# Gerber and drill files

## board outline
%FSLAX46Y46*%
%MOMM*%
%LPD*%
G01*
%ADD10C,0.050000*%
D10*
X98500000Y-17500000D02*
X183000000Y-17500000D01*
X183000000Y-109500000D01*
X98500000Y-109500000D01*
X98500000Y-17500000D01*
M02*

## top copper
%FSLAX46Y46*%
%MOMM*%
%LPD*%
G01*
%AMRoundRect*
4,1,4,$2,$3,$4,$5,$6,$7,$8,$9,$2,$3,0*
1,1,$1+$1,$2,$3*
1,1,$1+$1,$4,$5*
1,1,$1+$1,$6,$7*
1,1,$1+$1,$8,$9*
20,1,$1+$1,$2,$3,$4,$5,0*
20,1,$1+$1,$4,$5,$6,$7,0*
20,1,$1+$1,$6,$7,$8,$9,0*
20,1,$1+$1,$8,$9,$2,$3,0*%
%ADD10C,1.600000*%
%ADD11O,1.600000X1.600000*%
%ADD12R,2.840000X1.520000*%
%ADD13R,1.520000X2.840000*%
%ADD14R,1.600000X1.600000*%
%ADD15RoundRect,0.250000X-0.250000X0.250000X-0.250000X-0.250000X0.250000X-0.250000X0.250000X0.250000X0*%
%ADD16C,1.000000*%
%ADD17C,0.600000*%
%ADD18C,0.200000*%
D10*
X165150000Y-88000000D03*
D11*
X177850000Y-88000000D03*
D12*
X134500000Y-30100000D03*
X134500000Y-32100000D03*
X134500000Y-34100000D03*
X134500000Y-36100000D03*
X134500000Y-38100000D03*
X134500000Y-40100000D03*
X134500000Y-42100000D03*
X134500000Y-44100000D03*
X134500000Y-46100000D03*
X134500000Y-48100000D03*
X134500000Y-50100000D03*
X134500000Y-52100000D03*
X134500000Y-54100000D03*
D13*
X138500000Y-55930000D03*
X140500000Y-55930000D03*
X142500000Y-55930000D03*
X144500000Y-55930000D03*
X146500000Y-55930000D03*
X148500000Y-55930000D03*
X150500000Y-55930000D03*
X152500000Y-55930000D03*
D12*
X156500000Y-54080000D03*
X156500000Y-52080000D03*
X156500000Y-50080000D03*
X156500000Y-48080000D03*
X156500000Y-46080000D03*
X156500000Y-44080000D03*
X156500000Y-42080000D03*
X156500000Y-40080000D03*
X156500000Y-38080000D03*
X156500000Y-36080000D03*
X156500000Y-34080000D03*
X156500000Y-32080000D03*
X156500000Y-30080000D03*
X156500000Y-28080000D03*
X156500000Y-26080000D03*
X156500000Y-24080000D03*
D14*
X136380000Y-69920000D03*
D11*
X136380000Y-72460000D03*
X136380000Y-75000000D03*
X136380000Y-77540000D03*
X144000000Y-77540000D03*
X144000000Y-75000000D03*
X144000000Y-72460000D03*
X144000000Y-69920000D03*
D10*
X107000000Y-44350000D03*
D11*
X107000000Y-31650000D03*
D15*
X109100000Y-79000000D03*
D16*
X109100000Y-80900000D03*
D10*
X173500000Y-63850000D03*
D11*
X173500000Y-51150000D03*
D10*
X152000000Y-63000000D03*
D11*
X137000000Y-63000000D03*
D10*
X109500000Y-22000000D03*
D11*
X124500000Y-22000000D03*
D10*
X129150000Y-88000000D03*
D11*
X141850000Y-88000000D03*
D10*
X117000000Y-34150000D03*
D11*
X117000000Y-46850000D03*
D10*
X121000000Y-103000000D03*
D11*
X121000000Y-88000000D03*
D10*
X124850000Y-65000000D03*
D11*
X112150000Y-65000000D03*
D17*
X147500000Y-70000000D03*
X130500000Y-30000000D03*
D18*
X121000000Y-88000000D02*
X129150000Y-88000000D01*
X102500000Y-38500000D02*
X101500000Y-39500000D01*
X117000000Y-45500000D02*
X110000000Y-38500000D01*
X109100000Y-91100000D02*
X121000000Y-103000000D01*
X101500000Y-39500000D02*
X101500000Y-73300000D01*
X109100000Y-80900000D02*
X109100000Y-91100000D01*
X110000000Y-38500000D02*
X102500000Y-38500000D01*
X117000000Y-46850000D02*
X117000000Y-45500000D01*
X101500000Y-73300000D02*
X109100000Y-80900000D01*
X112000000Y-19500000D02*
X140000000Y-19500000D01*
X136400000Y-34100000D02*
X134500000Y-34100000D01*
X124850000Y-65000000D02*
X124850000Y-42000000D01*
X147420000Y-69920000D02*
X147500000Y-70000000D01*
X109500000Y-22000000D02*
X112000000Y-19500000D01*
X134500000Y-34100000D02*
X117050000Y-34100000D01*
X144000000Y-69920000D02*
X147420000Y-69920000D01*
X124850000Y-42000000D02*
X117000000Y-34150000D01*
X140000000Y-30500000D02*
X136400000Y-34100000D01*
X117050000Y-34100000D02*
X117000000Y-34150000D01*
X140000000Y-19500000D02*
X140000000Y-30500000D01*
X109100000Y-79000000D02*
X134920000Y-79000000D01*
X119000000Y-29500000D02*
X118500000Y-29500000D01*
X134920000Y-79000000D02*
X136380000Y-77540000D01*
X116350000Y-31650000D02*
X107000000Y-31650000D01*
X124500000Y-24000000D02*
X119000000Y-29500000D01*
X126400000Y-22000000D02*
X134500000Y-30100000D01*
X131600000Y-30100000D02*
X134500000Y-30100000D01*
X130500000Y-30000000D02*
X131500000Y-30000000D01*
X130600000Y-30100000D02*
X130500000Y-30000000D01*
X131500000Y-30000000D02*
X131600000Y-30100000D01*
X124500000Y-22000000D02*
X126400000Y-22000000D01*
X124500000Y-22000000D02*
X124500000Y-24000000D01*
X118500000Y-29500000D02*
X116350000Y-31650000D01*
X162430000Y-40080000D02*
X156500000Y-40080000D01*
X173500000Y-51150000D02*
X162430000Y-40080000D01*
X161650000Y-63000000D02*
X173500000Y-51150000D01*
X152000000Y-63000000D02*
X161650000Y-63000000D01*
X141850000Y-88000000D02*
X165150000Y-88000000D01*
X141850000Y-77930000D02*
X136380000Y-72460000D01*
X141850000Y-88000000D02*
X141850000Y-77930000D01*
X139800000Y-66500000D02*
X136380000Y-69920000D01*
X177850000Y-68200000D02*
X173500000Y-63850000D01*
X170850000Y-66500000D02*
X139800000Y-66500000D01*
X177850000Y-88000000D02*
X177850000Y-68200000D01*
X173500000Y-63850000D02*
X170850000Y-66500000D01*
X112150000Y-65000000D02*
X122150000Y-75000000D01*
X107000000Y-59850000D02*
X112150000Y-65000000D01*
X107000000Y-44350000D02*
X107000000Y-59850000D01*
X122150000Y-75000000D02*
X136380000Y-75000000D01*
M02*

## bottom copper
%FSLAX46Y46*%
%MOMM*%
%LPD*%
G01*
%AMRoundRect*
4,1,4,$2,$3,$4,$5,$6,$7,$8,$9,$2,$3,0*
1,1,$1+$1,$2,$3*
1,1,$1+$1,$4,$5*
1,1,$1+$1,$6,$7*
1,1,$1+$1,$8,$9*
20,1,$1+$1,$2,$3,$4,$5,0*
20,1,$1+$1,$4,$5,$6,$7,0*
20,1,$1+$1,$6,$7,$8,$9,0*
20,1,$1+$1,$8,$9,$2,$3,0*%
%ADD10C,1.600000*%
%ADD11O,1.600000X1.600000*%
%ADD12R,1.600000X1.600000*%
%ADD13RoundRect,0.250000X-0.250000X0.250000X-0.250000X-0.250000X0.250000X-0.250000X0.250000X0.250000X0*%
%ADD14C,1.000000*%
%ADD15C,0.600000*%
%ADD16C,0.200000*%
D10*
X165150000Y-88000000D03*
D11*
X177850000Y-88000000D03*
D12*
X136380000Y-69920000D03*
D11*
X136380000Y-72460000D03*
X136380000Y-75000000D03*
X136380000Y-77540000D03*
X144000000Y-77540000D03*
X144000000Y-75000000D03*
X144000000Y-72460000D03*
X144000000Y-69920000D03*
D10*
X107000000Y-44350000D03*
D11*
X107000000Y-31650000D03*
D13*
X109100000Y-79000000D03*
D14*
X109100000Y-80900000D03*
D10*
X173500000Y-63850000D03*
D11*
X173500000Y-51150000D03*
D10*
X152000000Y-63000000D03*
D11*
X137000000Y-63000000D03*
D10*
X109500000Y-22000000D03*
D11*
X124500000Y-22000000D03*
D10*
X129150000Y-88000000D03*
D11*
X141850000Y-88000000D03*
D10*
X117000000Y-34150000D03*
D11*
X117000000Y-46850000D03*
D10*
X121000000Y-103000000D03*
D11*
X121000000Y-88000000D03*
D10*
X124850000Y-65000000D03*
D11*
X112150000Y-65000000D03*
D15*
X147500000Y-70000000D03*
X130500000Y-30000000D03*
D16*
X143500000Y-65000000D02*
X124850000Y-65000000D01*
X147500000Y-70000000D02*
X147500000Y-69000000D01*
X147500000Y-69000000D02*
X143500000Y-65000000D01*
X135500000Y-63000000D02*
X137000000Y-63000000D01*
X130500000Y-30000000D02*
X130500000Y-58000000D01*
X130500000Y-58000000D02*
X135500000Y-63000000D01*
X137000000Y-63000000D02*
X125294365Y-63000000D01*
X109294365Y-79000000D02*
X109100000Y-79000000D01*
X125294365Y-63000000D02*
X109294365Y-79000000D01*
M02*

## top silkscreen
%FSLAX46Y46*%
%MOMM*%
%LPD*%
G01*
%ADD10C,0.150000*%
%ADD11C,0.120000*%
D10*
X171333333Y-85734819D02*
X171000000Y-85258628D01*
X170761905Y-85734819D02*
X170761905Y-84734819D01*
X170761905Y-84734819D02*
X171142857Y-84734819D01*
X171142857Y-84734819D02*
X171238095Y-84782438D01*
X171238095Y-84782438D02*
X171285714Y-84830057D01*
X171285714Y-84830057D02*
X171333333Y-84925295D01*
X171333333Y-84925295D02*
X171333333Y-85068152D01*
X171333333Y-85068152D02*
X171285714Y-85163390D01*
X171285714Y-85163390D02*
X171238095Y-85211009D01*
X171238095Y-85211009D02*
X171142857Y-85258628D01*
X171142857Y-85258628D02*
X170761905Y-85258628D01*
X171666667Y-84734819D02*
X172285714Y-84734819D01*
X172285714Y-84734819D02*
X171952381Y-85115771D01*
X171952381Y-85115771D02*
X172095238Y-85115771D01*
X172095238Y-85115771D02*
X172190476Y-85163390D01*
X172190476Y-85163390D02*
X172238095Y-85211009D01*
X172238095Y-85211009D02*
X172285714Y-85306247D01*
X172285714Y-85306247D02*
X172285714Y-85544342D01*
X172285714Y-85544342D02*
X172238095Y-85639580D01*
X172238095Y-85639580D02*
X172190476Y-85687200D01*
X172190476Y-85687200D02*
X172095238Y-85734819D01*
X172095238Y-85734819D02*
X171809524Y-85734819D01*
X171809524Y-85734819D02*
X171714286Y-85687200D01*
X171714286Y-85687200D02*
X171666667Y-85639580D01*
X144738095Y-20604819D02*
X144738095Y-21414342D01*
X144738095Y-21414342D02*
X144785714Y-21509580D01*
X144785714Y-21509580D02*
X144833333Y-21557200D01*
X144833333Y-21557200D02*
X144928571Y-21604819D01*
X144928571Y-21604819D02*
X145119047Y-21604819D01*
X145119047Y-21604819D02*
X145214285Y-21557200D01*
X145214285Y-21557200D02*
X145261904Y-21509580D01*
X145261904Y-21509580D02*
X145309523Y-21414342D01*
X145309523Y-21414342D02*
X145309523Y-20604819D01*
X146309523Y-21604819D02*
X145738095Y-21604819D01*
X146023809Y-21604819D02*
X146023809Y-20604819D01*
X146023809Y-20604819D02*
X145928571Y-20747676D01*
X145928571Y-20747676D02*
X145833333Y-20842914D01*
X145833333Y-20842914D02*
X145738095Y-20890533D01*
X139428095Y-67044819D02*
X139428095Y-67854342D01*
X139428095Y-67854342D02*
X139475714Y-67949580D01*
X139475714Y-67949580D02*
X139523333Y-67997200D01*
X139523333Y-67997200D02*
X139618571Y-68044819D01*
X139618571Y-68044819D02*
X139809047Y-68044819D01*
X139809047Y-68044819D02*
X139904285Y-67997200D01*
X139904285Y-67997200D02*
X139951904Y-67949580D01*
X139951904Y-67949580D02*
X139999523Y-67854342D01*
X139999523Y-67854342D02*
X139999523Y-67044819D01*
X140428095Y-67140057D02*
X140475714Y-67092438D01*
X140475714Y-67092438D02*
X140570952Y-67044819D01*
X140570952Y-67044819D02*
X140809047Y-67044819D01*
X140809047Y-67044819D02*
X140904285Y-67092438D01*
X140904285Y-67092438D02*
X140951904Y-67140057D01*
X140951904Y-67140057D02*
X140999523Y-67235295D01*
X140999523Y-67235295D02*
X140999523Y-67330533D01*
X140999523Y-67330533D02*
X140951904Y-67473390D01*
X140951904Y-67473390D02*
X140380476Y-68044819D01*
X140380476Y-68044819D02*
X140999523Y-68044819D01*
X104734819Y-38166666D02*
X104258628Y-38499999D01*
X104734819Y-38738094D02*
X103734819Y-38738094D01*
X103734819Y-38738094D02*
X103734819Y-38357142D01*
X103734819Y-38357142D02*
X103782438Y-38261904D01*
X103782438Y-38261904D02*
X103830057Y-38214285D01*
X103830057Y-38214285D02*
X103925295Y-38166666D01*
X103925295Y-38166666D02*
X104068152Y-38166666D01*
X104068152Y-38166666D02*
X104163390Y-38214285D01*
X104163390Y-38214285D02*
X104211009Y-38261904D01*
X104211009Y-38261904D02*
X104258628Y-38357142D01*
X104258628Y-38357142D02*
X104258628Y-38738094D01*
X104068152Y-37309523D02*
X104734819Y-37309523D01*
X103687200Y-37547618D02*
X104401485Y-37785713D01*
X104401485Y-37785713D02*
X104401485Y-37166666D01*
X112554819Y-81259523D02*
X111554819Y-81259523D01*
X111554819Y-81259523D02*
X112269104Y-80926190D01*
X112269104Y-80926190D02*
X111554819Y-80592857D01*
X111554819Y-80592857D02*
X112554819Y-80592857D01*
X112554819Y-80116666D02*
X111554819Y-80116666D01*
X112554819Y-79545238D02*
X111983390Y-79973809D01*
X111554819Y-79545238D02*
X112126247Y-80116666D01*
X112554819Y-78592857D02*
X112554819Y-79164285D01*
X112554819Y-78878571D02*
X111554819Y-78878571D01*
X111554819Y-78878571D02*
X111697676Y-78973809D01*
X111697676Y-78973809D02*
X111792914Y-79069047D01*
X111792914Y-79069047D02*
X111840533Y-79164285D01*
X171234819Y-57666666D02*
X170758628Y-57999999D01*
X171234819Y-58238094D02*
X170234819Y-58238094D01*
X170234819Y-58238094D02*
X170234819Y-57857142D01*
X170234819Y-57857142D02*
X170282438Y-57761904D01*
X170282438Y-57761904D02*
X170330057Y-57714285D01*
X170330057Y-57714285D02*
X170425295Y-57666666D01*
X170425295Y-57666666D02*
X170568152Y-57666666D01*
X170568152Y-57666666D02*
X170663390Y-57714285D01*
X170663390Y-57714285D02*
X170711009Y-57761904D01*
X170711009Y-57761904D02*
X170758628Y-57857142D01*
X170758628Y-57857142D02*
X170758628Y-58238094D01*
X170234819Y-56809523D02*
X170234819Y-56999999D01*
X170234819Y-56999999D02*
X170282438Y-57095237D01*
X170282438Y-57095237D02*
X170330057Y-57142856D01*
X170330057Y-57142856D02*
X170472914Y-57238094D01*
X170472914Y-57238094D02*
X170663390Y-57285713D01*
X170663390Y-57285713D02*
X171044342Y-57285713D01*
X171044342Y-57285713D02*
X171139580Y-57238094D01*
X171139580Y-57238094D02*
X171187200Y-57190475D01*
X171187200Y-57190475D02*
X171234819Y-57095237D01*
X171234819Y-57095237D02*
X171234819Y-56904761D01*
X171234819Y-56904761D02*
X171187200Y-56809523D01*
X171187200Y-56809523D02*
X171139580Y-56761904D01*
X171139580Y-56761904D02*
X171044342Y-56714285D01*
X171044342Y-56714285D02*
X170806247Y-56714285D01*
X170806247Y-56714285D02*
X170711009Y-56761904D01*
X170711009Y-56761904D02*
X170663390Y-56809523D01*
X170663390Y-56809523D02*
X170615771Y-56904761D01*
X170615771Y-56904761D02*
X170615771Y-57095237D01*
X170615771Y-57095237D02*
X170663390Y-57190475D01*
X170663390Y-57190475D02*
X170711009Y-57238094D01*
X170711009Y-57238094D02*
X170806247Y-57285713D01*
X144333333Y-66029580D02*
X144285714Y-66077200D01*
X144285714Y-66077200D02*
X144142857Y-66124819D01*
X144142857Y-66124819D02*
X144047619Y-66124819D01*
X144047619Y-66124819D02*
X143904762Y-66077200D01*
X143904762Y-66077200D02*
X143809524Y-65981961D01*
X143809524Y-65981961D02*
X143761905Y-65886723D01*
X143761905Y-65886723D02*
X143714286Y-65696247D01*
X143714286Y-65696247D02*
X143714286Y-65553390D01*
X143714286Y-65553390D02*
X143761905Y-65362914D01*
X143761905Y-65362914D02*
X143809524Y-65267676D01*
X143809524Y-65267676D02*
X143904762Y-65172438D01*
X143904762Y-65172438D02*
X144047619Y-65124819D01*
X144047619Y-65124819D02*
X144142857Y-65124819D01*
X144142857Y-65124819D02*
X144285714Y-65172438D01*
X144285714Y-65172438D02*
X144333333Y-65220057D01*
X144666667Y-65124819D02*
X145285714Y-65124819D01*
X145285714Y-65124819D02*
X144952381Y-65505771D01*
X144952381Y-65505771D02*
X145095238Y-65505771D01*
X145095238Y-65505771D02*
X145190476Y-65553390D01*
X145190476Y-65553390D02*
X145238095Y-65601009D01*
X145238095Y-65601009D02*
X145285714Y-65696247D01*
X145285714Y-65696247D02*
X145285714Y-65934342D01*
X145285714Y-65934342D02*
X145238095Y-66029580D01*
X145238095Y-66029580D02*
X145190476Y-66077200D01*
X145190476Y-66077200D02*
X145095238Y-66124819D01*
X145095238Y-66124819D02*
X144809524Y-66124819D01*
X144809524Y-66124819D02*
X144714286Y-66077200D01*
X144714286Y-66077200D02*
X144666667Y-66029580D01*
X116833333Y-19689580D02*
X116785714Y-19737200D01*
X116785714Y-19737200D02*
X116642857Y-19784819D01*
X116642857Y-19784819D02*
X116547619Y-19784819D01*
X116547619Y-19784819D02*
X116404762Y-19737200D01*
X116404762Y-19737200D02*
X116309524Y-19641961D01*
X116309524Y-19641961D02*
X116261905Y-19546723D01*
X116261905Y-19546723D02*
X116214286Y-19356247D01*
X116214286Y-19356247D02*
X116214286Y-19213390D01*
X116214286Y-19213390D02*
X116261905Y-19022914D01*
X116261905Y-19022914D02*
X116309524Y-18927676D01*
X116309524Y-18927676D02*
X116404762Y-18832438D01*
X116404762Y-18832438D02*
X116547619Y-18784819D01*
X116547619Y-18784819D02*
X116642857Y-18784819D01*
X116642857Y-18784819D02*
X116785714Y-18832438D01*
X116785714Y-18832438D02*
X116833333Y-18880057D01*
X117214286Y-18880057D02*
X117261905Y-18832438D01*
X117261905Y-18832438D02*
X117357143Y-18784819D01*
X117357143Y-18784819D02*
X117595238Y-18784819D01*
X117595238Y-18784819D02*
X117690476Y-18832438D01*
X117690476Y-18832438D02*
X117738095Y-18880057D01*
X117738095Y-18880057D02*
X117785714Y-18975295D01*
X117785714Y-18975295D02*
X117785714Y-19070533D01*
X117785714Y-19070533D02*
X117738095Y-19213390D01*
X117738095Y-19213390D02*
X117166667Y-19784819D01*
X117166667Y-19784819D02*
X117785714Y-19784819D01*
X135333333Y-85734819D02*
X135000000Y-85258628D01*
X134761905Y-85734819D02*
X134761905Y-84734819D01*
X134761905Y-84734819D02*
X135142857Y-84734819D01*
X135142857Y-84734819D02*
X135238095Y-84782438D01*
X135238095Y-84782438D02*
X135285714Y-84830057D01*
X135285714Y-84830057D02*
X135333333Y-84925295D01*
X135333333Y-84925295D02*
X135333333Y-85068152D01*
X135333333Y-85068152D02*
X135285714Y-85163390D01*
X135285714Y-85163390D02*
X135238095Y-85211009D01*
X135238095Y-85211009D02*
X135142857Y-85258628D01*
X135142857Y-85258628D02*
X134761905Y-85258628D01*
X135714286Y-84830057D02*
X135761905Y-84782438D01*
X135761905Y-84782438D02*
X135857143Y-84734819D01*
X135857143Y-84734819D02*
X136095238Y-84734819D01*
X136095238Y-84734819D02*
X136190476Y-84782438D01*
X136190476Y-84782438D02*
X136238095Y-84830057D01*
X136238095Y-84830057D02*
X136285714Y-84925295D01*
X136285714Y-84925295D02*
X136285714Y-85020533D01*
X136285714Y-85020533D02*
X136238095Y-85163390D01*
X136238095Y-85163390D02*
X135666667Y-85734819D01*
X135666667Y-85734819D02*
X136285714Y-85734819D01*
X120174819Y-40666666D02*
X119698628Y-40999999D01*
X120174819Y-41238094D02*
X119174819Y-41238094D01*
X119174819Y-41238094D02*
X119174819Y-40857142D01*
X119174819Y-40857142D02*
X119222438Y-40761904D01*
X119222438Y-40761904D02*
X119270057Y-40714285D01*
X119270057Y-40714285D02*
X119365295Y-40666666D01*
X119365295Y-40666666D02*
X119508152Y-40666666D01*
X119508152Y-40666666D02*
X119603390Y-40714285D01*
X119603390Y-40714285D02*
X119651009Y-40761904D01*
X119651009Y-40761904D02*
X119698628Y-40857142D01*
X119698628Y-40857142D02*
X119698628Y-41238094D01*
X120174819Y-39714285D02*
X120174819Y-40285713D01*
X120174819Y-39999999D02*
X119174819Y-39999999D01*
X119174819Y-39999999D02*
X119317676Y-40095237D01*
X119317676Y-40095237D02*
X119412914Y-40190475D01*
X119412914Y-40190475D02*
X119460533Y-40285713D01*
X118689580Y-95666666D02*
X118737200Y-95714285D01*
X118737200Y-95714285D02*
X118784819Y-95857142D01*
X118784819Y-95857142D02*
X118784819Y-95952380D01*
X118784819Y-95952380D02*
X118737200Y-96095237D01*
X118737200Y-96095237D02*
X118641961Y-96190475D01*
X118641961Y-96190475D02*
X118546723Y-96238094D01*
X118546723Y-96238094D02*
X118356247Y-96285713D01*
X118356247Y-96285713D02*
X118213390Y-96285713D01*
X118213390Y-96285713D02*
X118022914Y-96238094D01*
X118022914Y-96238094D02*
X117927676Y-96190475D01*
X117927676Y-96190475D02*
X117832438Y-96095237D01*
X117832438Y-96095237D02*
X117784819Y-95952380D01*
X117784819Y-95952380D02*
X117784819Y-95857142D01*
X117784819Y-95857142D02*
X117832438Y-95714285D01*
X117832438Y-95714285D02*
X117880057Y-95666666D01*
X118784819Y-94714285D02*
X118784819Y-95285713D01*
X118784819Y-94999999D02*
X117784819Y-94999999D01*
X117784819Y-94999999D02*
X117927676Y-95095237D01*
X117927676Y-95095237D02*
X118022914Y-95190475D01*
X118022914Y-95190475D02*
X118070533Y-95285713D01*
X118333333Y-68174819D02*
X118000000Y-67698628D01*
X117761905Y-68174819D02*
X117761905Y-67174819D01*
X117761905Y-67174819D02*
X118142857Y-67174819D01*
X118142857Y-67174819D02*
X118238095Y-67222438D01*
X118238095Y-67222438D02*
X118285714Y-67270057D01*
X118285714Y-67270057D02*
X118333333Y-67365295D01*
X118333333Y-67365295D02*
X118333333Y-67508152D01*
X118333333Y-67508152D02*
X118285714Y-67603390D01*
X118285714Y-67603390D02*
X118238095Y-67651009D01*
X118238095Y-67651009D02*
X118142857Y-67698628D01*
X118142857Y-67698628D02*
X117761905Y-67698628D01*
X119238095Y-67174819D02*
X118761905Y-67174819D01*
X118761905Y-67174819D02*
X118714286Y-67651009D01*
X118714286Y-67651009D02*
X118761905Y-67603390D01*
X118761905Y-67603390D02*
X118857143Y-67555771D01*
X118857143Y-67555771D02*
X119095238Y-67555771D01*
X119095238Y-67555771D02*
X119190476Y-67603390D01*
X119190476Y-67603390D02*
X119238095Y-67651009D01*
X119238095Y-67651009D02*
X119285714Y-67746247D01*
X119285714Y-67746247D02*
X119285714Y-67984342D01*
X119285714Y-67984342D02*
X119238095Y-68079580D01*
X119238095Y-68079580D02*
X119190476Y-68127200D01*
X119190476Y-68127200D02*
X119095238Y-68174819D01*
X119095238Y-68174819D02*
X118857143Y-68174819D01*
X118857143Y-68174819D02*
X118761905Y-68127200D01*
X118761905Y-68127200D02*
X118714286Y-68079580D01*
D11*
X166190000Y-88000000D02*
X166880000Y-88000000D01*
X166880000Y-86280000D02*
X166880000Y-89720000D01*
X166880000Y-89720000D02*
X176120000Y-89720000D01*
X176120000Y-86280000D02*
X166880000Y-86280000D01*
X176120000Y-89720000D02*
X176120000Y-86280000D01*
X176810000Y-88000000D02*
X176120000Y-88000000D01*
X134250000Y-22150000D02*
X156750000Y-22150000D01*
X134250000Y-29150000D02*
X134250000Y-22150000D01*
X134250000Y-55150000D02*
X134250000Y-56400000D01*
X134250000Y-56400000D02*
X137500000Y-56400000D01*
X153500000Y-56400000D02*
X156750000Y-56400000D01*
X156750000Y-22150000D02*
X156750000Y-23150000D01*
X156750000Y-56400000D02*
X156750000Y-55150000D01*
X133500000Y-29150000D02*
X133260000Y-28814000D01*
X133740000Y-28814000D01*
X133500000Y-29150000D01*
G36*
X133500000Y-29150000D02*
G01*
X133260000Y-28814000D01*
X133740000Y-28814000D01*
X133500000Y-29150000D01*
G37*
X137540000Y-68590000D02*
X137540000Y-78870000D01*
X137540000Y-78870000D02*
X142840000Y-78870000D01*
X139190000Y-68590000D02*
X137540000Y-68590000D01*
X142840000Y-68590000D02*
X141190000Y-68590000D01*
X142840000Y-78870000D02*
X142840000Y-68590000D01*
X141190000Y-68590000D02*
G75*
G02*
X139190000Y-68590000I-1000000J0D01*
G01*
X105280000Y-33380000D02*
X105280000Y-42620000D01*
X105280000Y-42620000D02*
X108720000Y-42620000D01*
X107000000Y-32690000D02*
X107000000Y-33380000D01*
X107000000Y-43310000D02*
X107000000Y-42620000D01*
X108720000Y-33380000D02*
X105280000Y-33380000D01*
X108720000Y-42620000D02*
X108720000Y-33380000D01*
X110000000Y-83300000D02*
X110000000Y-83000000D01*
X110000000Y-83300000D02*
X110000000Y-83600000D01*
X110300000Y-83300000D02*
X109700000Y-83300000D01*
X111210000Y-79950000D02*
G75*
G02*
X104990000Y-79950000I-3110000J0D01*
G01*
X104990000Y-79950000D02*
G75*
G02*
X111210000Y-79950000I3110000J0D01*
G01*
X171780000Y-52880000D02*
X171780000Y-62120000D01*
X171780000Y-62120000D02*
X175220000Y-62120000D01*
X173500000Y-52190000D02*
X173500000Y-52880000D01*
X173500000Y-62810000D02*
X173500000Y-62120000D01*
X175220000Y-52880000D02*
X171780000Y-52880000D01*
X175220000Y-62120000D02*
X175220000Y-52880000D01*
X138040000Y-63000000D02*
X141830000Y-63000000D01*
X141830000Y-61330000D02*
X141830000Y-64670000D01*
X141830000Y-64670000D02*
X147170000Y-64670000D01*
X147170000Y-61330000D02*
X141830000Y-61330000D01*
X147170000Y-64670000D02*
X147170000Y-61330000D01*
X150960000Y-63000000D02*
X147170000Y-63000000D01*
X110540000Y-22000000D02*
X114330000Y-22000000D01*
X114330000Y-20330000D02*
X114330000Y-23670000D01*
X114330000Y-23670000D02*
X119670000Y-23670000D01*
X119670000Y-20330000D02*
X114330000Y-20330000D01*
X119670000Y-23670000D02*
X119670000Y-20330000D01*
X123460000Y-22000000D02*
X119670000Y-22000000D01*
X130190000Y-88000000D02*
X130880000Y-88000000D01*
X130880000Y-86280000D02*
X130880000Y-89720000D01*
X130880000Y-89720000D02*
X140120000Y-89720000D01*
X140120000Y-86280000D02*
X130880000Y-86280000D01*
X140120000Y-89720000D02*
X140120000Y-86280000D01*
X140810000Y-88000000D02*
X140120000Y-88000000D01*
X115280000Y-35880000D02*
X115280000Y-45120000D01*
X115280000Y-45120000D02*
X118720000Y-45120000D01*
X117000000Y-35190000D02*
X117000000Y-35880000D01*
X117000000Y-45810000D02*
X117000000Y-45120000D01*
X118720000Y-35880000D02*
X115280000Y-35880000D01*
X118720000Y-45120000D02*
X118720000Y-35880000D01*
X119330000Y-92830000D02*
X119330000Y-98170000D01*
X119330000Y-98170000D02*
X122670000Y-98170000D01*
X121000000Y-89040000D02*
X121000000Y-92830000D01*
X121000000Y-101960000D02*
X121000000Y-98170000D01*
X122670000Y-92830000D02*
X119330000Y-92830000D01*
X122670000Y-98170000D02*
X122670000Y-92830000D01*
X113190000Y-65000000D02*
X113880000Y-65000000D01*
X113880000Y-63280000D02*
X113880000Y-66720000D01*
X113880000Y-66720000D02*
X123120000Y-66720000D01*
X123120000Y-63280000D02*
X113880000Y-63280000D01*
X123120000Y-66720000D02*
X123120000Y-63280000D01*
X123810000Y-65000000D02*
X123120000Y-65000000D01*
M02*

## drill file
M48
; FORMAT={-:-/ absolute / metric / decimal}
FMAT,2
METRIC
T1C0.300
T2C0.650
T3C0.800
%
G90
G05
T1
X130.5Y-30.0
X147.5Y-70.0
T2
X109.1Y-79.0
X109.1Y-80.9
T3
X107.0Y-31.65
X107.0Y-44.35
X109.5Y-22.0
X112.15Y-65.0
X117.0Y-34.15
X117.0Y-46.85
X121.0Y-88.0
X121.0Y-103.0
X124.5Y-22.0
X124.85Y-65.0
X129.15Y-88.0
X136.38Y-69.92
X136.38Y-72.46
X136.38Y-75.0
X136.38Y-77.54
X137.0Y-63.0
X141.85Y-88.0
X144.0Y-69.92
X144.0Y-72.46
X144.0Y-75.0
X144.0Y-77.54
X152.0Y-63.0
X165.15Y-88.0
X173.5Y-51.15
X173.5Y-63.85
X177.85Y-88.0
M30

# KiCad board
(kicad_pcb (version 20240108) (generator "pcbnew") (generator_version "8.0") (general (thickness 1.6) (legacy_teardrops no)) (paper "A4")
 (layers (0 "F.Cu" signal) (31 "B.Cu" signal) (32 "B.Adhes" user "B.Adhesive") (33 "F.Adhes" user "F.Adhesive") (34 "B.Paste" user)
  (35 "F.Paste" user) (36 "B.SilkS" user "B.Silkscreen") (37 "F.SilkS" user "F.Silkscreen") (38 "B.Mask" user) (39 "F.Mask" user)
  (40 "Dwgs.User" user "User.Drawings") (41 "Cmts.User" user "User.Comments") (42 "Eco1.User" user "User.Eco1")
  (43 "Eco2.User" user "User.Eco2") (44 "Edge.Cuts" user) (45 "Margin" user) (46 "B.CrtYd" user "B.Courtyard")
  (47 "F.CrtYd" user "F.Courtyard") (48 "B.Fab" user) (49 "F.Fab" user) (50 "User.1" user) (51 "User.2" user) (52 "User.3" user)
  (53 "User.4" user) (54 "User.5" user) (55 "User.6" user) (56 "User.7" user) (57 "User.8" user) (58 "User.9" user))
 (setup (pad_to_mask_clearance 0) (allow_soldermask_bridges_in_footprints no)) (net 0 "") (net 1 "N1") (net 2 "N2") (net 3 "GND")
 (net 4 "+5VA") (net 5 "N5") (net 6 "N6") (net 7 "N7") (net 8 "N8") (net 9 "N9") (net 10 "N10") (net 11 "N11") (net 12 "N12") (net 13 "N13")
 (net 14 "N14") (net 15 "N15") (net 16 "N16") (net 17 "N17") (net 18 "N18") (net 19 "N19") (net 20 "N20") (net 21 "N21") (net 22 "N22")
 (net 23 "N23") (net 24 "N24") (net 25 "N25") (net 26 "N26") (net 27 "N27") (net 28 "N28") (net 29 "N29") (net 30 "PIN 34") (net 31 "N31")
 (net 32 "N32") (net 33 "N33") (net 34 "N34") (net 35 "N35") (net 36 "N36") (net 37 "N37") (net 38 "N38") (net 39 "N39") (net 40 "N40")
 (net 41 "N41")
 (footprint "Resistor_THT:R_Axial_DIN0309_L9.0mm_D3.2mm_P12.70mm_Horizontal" (layer "F.Cu") (at 165.15 88)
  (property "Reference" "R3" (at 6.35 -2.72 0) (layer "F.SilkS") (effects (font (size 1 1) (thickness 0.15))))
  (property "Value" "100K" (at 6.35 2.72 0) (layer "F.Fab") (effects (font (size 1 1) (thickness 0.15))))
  (fp_line (start 1.04 0) (end 1.73 0) (stroke (width 0.12) (type solid)) (layer "F.SilkS"))
  (fp_line (start 1.73 -1.72) (end 1.73 1.72) (stroke (width 0.12) (type solid)) (layer "F.SilkS"))
  (fp_line (start 1.73 1.72) (end 10.97 1.72) (stroke (width 0.12) (type solid)) (layer "F.SilkS"))
  (fp_line (start 10.97 -1.72) (end 1.73 -1.72) (stroke (width 0.12) (type solid)) (layer "F.SilkS"))
  (fp_line (start 10.97 1.72) (end 10.97 -1.72) (stroke (width 0.12) (type solid)) (layer "F.SilkS"))
  (fp_line (start 11.66 0) (end 10.97 0) (stroke (width 0.12) (type solid)) (layer "F.SilkS"))
  (pad "1" thru_hole circle (at 0 0) (size 1.6 1.6) (drill 0.8) (layers "*.Cu" "*.Mask") (remove_unused_layers no) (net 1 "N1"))
  (pad "2" thru_hole oval (at 12.7 0) (size 1.6 1.6) (drill 0.8) (layers "*.Cu" "*.Mask") (remove_unused_layers no) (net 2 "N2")))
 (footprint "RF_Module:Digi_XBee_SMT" (layer "F.Cu") (at 145.5 40)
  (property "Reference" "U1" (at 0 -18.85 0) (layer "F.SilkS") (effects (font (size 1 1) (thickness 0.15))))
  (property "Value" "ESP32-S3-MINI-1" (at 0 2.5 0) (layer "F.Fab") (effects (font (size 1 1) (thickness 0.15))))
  (fp_line (start -11.25 -17.85) (end 11.25 -17.85) (stroke (width 0.12) (type solid)) (layer "F.SilkS"))
  (fp_line (start -11.25 -10.85) (end -11.25 -17.85) (stroke (width 0.12) (type solid)) (layer "F.SilkS"))
  (fp_line (start -11.25 15.15) (end -11.25 16.4) (stroke (width 0.12) (type solid)) (layer "F.SilkS"))
  (fp_line (start -11.25 16.4) (end -8 16.4) (stroke (width 0.12) (type solid)) (layer "F.SilkS"))
  (fp_line (start 8 16.4) (end 11.25 16.4) (stroke (width 0.12) (type solid)) (layer "F.SilkS"))
  (fp_line (start 11.25 -17.85) (end 11.25 -16.85) (stroke (width 0.12) (type solid)) (layer "F.SilkS"))
  (fp_line (start 11.25 16.4) (end 11.25 15.15) (stroke (width 0.12) (type solid)) (layer "F.SilkS"))
  (fp_poly
   (pts (xy -12 -10.85) (xy -12.24 -11.186) (xy -11.76 -11.186) (xy -12 -10.85)) (stroke (width 0.12) (type solid)) (fill solid)
   (layer "F.SilkS"))
  (pad "1" smd rect (at -11 -9.9) (size 2.84 1.52) (layers "F.Cu" "F.Paste" "F.Mask") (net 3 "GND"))
  (pad "2" smd rect (at -11 -7.9) (size 2.84 1.52) (layers "F.Cu" "F.Paste" "F.Mask") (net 3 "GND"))
  (pad "3" smd rect (at -11 -5.9) (size 2.84 1.52) (layers "F.Cu" "F.Paste" "F.Mask") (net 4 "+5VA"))
  (pad "4" smd rect (at -11 -3.9) (size 2.84 1.52) (layers "F.Cu" "F.Paste" "F.Mask") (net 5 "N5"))
  (pad "5" smd rect (at -11 -1.9) (size 2.84 1.52) (layers "F.Cu" "F.Paste" "F.Mask") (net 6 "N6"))
  (pad "6" smd rect (at -11 0.1) (size 2.84 1.52) (layers "F.Cu" "F.Paste" "F.Mask") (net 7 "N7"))
  (pad "7" smd rect (at -11 2.1) (size 2.84 1.52) (layers "F.Cu" "F.Paste" "F.Mask") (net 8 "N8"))
  (pad "8" smd rect (at -11 4.1) (size 2.84 1.52) (layers "F.Cu" "F.Paste" "F.Mask") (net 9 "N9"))
  (pad "9" smd rect (at -11 6.1) (size 2.84 1.52) (layers "F.Cu" "F.Paste" "F.Mask") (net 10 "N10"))
  (pad "10" smd rect (at -11 8.1) (size 2.84 1.52) (layers "F.Cu" "F.Paste" "F.Mask") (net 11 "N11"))
  (pad "11" smd rect (at -11 10.1) (size 2.84 1.52) (layers "F.Cu" "F.Paste" "F.Mask") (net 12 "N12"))
  (pad "12" smd rect (at -11 12.1) (size 2.84 1.52) (layers "F.Cu" "F.Paste" "F.Mask") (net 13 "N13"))
  (pad "13" smd rect (at -11 14.1) (size 2.84 1.52) (layers "F.Cu" "F.Paste" "F.Mask") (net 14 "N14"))
  (pad "14" smd rect (at -7 15.93 90) (size 2.84 1.52) (layers "F.Cu" "F.Paste" "F.Mask") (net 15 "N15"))
  (pad "15" smd rect (at -5 15.93 90) (size 2.84 1.52) (layers "F.Cu" "F.Paste" "F.Mask") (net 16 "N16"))
  (pad "16" smd rect (at -3 15.93 90) (size 2.84 1.52) (layers "F.Cu" "F.Paste" "F.Mask") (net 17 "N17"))
  (pad "17" smd rect (at -1 15.93 90) (size 2.84 1.52) (layers "F.Cu" "F.Paste" "F.Mask") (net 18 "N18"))
  (pad "18" smd rect (at 1 15.93 90) (size 2.84 1.52) (layers "F.Cu" "F.Paste" "F.Mask") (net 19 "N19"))
  (pad "19" smd rect (at 3 15.93 90) (size 2.84 1.52) (layers "F.Cu" "F.Paste" "F.Mask") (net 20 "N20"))
  (pad "20" smd rect (at 5 15.93 90) (size 2.84 1.52) (layers "F.Cu" "F.Paste" "F.Mask") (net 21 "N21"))
  (pad "21" smd rect (at 7 15.93 90) (size 2.84 1.52) (layers "F.Cu" "F.Paste" "F.Mask") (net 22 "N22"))
  (pad "22" smd rect (at 11 14.08) (size 2.84 1.52) (layers "F.Cu" "F.Paste" "F.Mask") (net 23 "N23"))
  (pad "23" smd rect (at 11 12.08) (size 2.84 1.52) (layers "F.Cu" "F.Paste" "F.Mask") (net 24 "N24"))
  (pad "24" smd rect (at 11 10.08) (size 2.84 1.52) (layers "F.Cu" "F.Paste" "F.Mask") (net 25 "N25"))
  (pad "25" smd rect (at 11 8.08) (size 2.84 1.52) (layers "F.Cu" "F.Paste" "F.Mask") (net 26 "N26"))
  (pad "26" smd rect (at 11 6.08) (size 2.84 1.52) (layers "F.Cu" "F.Paste" "F.Mask") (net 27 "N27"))
  (pad "27" smd rect (at 11 4.08) (size 2.84 1.52) (layers "F.Cu" "F.Paste" "F.Mask") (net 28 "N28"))
  (pad "28" smd rect (at 11 2.08) (size 2.84 1.52) (layers "F.Cu" "F.Paste" "F.Mask") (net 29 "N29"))
  (pad "29" smd rect (at 11 0.08) (size 2.84 1.52) (layers "F.Cu" "F.Paste" "F.Mask") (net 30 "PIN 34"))
  (pad "30" smd rect (at 11 -1.92) (size 2.84 1.52) (layers "F.Cu" "F.Paste" "F.Mask") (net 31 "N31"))
  (pad "31" smd rect (at 11 -3.92) (size 2.84 1.52) (layers "F.Cu" "F.Paste" "F.Mask") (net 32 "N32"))
  (pad "32" smd rect (at 11 -5.92) (size 2.84 1.52) (layers "F.Cu" "F.Paste" "F.Mask") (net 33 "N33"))
  (pad "33" smd rect (at 11 -7.92) (size 2.84 1.52) (layers "F.Cu" "F.Paste" "F.Mask") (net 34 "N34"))
  (pad "34" smd rect (at 11 -9.92) (size 2.84 1.52) (layers "F.Cu" "F.Paste" "F.Mask") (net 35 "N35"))
  (pad "35" smd rect (at 11 -11.92) (size 2.84 1.52) (layers "F.Cu" "F.Paste" "F.Mask") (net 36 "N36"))
  (pad "36" smd rect (at 11 -13.92) (size 2.84 1.52) (layers "F.Cu" "F.Paste" "F.Mask") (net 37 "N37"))
  (pad "37" smd rect (at 11 -15.92) (size 2.84 1.52) (layers "F.Cu" "F.Paste" "F.Mask") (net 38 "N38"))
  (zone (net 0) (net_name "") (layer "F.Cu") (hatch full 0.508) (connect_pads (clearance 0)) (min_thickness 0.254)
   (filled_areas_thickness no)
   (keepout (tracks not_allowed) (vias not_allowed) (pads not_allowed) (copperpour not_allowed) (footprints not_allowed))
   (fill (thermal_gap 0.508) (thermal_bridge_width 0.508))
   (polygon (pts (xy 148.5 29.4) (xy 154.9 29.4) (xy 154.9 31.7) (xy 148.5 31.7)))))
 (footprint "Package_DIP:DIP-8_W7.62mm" (layer "F.Cu") (at 136.38 69.92)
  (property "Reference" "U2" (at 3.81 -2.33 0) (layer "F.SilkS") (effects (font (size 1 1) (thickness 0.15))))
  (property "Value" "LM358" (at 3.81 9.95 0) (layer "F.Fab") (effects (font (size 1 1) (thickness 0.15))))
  (fp_line (start 1.16 -1.33) (end 1.16 8.95) (stroke (width 0.12) (type solid)) (layer "F.SilkS"))
  (fp_line (start 1.16 8.95) (end 6.46 8.95) (stroke (width 0.12) (type solid)) (layer "F.SilkS"))
  (fp_line (start 2.81 -1.33) (end 1.16 -1.33) (stroke (width 0.12) (type solid)) (layer "F.SilkS"))
  (fp_line (start 6.46 -1.33) (end 4.81 -1.33) (stroke (width 0.12) (type solid)) (layer "F.SilkS"))
  (fp_line (start 6.46 8.95) (end 6.46 -1.33) (stroke (width 0.12) (type solid)) (layer "F.SilkS"))
  (fp_arc (start 4.81 -1.33) (mid 3.81 -0.33) (end 2.81 -1.33) (stroke (width 0.12) (type solid)) (layer "F.SilkS"))
  (pad "1" thru_hole rect (at 0 0) (size 1.6 1.6) (drill 0.8) (layers "*.Cu" "*.Mask") (remove_unused_layers no) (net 2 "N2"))
  (pad "2" thru_hole oval (at 0 2.54) (size 1.6 1.6) (drill 0.8) (layers "*.Cu" "*.Mask") (remove_unused_layers no) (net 1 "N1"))
  (pad "3" thru_hole oval (at 0 5.08) (size 1.6 1.6) (drill 0.8) (layers "*.Cu" "*.Mask") (remove_unused_layers no) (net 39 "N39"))
  (pad "4" thru_hole oval (at 0 7.62) (size 1.6 1.6) (drill 0.8) (layers "*.Cu" "*.Mask") (remove_unused_layers no) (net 3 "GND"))
  (pad "5" thru_hole oval (at 7.62 7.62) (size 1.6 1.6) (drill 0.8) (layers "*.Cu" "*.Mask") (remove_unused_layers no))
  (pad "6" thru_hole oval (at 7.62 5.08) (size 1.6 1.6) (drill 0.8) (layers "*.Cu" "*.Mask") (remove_unused_layers no))
  (pad "7" thru_hole oval (at 7.62 2.54) (size 1.6 1.6) (drill 0.8) (layers "*.Cu" "*.Mask") (remove_unused_layers no))
  (pad "8" thru_hole oval (at 7.62 0) (size 1.6 1.6) (drill 0.8) (layers "*.Cu" "*.Mask") (remove_unused_layers no) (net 4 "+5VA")))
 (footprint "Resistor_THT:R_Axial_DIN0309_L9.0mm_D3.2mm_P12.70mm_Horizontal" (layer "F.Cu") (at 107 44.35 90)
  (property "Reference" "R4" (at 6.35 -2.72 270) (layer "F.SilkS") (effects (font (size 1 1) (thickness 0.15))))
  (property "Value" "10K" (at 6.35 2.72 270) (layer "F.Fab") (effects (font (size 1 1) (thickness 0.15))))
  (fp_line (start 10.97 -1.72) (end 1.73 -1.72) (stroke (width 0.12) (type solid)) (layer "F.SilkS"))
  (fp_line (start 1.73 -1.72) (end 1.73 1.72) (stroke (width 0.12) (type solid)) (layer "F.SilkS"))
  (fp_line (start 11.66 0) (end 10.97 0) (stroke (width 0.12) (type solid)) (layer "F.SilkS"))
  (fp_line (start 1.04 0) (end 1.73 0) (stroke (width 0.12) (type solid)) (layer "F.SilkS"))
  (fp_line (start 10.97 1.72) (end 10.97 -1.72) (stroke (width 0.12) (type solid)) (layer "F.SilkS"))
  (fp_line (start 1.73 1.72) (end 10.97 1.72) (stroke (width 0.12) (type solid)) (layer "F.SilkS"))
  (pad "1" thru_hole circle (at 0 0 90) (size 1.6 1.6) (drill 0.8) (layers "*.Cu" "*.Mask") (remove_unused_layers no) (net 39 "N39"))
  (pad "2" thru_hole oval (at 12.7 0 90) (size 1.6 1.6) (drill 0.8) (layers "*.Cu" "*.Mask") (remove_unused_layers no) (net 3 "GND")))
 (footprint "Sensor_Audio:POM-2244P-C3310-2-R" (layer "F.Cu") (at 109.1 79 -90)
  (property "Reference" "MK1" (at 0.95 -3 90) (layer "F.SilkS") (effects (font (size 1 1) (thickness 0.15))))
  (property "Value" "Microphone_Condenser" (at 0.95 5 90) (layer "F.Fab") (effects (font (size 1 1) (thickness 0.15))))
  (fp_line (start 4.3 -0.9) (end 4 -0.9) (stroke (width 0.12) (type default)) (layer "F.SilkS"))
  (fp_line (start 4.3 -0.9) (end 4.6 -0.9) (stroke (width 0.12) (type default)) (layer "F.SilkS"))
  (fp_line (start 4.3 -1.2) (end 4.3 -0.6) (stroke (width 0.12) (type default)) (layer "F.SilkS"))
  (fp_circle (center 0.95 1) (end 4.06 1) (stroke (width 0.12) (type default)) (fill none) (layer "F.SilkS"))
  (pad "1" thru_hole roundrect (at 0 0 270) (size 1 1) (drill 0.65) (layers "*.Cu" "*.Mask") (remove_unused_layers no)
   (roundrect_rratio 0.25) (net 3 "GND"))
  (pad "2" thru_hole circle (at 1.9 0 270) (size 1 1) (drill 0.65) (layers "*.Cu" "*.Mask") (remove_unused_layers no) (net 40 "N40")))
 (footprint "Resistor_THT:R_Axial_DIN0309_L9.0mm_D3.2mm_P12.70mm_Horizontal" (layer "F.Cu") (at 173.5 63.85 90)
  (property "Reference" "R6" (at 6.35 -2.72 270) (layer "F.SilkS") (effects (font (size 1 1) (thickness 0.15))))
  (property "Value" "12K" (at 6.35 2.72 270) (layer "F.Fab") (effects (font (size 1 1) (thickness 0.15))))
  (fp_line (start 10.97 -1.72) (end 1.73 -1.72) (stroke (width 0.12) (type solid)) (layer "F.SilkS"))
  (fp_line (start 1.73 -1.72) (end 1.73 1.72) (stroke (width 0.12) (type solid)) (layer "F.SilkS"))
  (fp_line (start 11.66 0) (end 10.97 0) (stroke (width 0.12) (type solid)) (layer "F.SilkS"))
  (fp_line (start 1.04 0) (end 1.73 0) (stroke (width 0.12) (type solid)) (layer "F.SilkS"))
  (fp_line (start 10.97 1.72) (end 10.97 -1.72) (stroke (width 0.12) (type solid)) (layer "F.SilkS"))
  (fp_line (start 1.73 1.72) (end 10.97 1.72) (stroke (width 0.12) (type solid)) (layer "F.SilkS"))
  (pad "1" thru_hole circle (at 0 0 90) (size 1.6 1.6) (drill 0.8) (layers "*.Cu" "*.Mask") (remove_unused_layers no) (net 2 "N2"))
  (pad "2" thru_hole oval (at 12.7 0 90) (size 1.6 1.6) (drill 0.8) (layers "*.Cu" "*.Mask") (remove_unused_layers no) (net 30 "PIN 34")))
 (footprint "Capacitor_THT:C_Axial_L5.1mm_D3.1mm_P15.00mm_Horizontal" (layer "F.Cu") (at 152 63 180)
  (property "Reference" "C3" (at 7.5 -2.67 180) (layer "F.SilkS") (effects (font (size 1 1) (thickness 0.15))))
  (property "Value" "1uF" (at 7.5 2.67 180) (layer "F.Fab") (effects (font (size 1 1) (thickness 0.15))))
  (fp_line (start 13.96 0) (end 10.17 0) (stroke (width 0.12) (type solid)) (layer "F.SilkS"))
  (fp_line (start 10.17 1.67) (end 10.17 -1.67) (stroke (width 0.12) (type solid)) (layer "F.SilkS"))
  (fp_line (start 10.17 -1.67) (end 4.83 -1.67) (stroke (width 0.12) (type solid)) (layer "F.SilkS"))
  (fp_line (start 4.83 1.67) (end 10.17 1.67) (stroke (width 0.12) (type solid)) (layer "F.SilkS"))
  (fp_line (start 4.83 -1.67) (end 4.83 1.67) (stroke (width 0.12) (type solid)) (layer "F.SilkS"))
  (fp_line (start 1.04 0) (end 4.83 0) (stroke (width 0.12) (type solid)) (layer "F.SilkS"))
  (pad "1" thru_hole circle (at 0 0 180) (size 1.6 1.6) (drill 0.8) (layers "*.Cu" "*.Mask") (remove_unused_layers no) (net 30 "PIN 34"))
  (pad "2" thru_hole oval (at 15 0 180) (size 1.6 1.6) (drill 0.8) (layers "*.Cu" "*.Mask") (remove_unused_layers no) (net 3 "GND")))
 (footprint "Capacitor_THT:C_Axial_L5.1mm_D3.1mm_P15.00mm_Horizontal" (layer "F.Cu") (at 109.5 22)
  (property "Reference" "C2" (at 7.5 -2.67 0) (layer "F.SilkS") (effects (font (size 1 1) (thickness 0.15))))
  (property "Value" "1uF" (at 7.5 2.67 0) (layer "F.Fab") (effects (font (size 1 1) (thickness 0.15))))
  (fp_line (start 1.04 0) (end 4.83 0) (stroke (width 0.12) (type solid)) (layer "F.SilkS"))
  (fp_line (start 4.83 -1.67) (end 4.83 1.67) (stroke (width 0.12) (type solid)) (layer "F.SilkS"))
  (fp_line (start 4.83 1.67) (end 10.17 1.67) (stroke (width 0.12) (type solid)) (layer "F.SilkS"))
  (fp_line (start 10.17 -1.67) (end 4.83 -1.67) (stroke (width 0.12) (type solid)) (layer "F.SilkS"))
  (fp_line (start 10.17 1.67) (end 10.17 -1.67) (stroke (width 0.12) (type solid)) (layer "F.SilkS"))
  (fp_line (start 13.96 0) (end 10.17 0) (stroke (width 0.12) (type solid)) (layer "F.SilkS"))
  (pad "1" thru_hole circle (at 0 0) (size 1.6 1.6) (drill 0.8) (layers "*.Cu" "*.Mask") (remove_unused_layers no) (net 4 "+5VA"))
  (pad "2" thru_hole oval (at 15 0) (size 1.6 1.6) (drill 0.8) (layers "*.Cu" "*.Mask") (remove_unused_layers no) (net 3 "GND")))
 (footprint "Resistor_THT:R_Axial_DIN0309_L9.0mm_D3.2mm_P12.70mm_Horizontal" (layer "F.Cu") (at 129.15 88)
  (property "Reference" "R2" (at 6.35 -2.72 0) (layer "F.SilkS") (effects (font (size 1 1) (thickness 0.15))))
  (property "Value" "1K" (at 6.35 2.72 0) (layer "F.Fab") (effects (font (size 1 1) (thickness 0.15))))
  (fp_line (start 1.04 0) (end 1.73 0) (stroke (width 0.12) (type solid)) (layer "F.SilkS"))
  (fp_line (start 1.73 -1.72) (end 1.73 1.72) (stroke (width 0.12) (type solid)) (layer "F.SilkS"))
  (fp_line (start 1.73 1.72) (end 10.97 1.72) (stroke (width 0.12) (type solid)) (layer "F.SilkS"))
  (fp_line (start 10.97 -1.72) (end 1.73 -1.72) (stroke (width 0.12) (type solid)) (layer "F.SilkS"))
  (fp_line (start 10.97 1.72) (end 10.97 -1.72) (stroke (width 0.12) (type solid)) (layer "F.SilkS"))
  (fp_line (start 11.66 0) (end 10.97 0) (stroke (width 0.12) (type solid)) (layer "F.SilkS"))
  (pad "1" thru_hole circle (at 0 0) (size 1.6 1.6) (drill 0.8) (layers "*.Cu" "*.Mask") (remove_unused_layers no) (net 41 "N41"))
  (pad "2" thru_hole oval (at 12.7 0) (size 1.6 1.6) (drill 0.8) (layers "*.Cu" "*.Mask") (remove_unused_layers no) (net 1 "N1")))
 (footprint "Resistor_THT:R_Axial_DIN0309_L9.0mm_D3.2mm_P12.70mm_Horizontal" (layer "F.Cu") (at 117 34.15 -90)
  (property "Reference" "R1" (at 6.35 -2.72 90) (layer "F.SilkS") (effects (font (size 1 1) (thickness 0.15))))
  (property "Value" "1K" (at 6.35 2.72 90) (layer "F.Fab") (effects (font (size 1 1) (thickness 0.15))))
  (fp_line (start 1.73 1.72) (end 10.97 1.72) (stroke (width 0.12) (type solid)) (layer "F.SilkS"))
  (fp_line (start 10.97 1.72) (end 10.97 -1.72) (stroke (width 0.12) (type solid)) (layer "F.SilkS"))
  (fp_line (start 1.04 0) (end 1.73 0) (stroke (width 0.12) (type solid)) (layer "F.SilkS"))
  (fp_line (start 11.66 0) (end 10.97 0) (stroke (width 0.12) (type solid)) (layer "F.SilkS"))
  (fp_line (start 1.73 -1.72) (end 1.73 1.72) (stroke (width 0.12) (type solid)) (layer "F.SilkS"))
  (fp_line (start 10.97 -1.72) (end 1.73 -1.72) (stroke (width 0.12) (type solid)) (layer "F.SilkS"))
  (pad "1" thru_hole circle (at 0 0 270) (size 1.6 1.6) (drill 0.8) (layers "*.Cu" "*.Mask") (remove_unused_layers no) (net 4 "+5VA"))
  (pad "2" thru_hole oval (at 12.7 0 270) (size 1.6 1.6) (drill 0.8) (layers "*.Cu" "*.Mask") (remove_unused_layers no) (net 40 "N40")))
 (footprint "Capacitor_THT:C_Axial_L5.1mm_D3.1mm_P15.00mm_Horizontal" (layer "F.Cu") (at 121 103 90)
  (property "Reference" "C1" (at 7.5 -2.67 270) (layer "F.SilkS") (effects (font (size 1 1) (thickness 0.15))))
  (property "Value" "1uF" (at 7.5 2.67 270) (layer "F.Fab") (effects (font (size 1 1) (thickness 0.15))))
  (fp_line (start 10.17 -1.67) (end 4.83 -1.67) (stroke (width 0.12) (type solid)) (layer "F.SilkS"))
  (fp_line (start 4.83 -1.67) (end 4.83 1.67) (stroke (width 0.12) (type solid)) (layer "F.SilkS"))
  (fp_line (start 13.96 0) (end 10.17 0) (stroke (width 0.12) (type solid)) (layer "F.SilkS"))
  (fp_line (start 1.04 0) (end 4.83 0) (stroke (width 0.12) (type solid)) (layer "F.SilkS"))
  (fp_line (start 10.17 1.67) (end 10.17 -1.67) (stroke (width 0.12) (type solid)) (layer "F.SilkS"))
  (fp_line (start 4.83 1.67) (end 10.17 1.67) (stroke (width 0.12) (type solid)) (layer "F.SilkS"))
  (pad "1" thru_hole circle (at 0 0 90) (size 1.6 1.6) (drill 0.8) (layers "*.Cu" "*.Mask") (remove_unused_layers no) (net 40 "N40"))
  (pad "2" thru_hole oval (at 15 0 90) (size 1.6 1.6) (drill 0.8) (layers "*.Cu" "*.Mask") (remove_unused_layers no) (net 41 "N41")))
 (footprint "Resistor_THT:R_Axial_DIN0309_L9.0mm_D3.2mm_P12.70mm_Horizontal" (layer "F.Cu") (at 124.85 65 180)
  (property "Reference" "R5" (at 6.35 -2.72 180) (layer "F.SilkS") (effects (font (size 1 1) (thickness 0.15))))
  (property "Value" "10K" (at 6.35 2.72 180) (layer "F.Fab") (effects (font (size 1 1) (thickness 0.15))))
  (fp_line (start 11.66 0) (end 10.97 0) (stroke (width 0.12) (type solid)) (layer "F.SilkS"))
  (fp_line (start 10.97 1.72) (end 10.97 -1.72) (stroke (width 0.12) (type solid)) (layer "F.SilkS"))
  (fp_line (start 10.97 -1.72) (end 1.73 -1.72) (stroke (width 0.12) (type solid)) (layer "F.SilkS"))
  (fp_line (start 1.73 1.72) (end 10.97 1.72) (stroke (width 0.12) (type solid)) (layer "F.SilkS"))
  (fp_line (start 1.73 -1.72) (end 1.73 1.72) (stroke (width 0.12) (type solid)) (layer "F.SilkS"))
  (fp_line (start 1.04 0) (end 1.73 0) (stroke (width 0.12) (type solid)) (layer "F.SilkS"))
  (pad "1" thru_hole circle (at 0 0 180) (size 1.6 1.6) (drill 0.8) (layers "*.Cu" "*.Mask") (remove_unused_layers no) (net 4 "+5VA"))
  (pad "2" thru_hole oval (at 12.7 0 180) (size 1.6 1.6) (drill 0.8) (layers "*.Cu" "*.Mask") (remove_unused_layers no) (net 39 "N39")))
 (gr_rect (start 98.5 17.5) (end 183 109.5) (stroke (width 0.05) (type default)) (fill none) (layer "Edge.Cuts"))
 (segment (start 121 88) (end 129.15 88) (width 0.2) (layer "F.Cu") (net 41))
 (segment (start 102.5 38.5) (end 101.5 39.5) (width 0.2) (layer "F.Cu") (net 40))
 (segment (start 117 45.5) (end 110 38.5) (width 0.2) (layer "F.Cu") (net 40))
 (segment (start 109.1 91.1) (end 121 103) (width 0.2) (layer "F.Cu") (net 40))
 (segment (start 101.5 39.5) (end 101.5 73.3) (width 0.2) (layer "F.Cu") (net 40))
 (segment (start 109.1 80.9) (end 109.1 91.1) (width 0.2) (layer "F.Cu") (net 40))
 (segment (start 110 38.5) (end 102.5 38.5) (width 0.2) (layer "F.Cu") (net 40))
 (segment (start 117 46.85) (end 117 45.5) (width 0.2) (layer "F.Cu") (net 40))
 (segment (start 101.5 73.3) (end 109.1 80.9) (width 0.2) (layer "F.Cu") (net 40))
 (segment (start 112 19.5) (end 140 19.5) (width 0.2) (layer "F.Cu") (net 4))
 (segment (start 136.4 34.1) (end 134.5 34.1) (width 0.2) (layer "F.Cu") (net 4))
 (segment (start 124.85 65) (end 124.85 42) (width 0.2) (layer "F.Cu") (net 4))
 (segment (start 147.42 69.92) (end 147.5 70) (width 0.2) (layer "F.Cu") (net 4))
 (segment (start 109.5 22) (end 112 19.5) (width 0.2) (layer "F.Cu") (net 4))
 (segment (start 134.5 34.1) (end 117.05 34.1) (width 0.2) (layer "F.Cu") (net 4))
 (segment (start 144 69.92) (end 147.42 69.92) (width 0.2) (layer "F.Cu") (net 4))
 (segment (start 124.85 42) (end 117 34.15) (width 0.2) (layer "F.Cu") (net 4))
 (segment (start 140 30.5) (end 136.4 34.1) (width 0.2) (layer "F.Cu") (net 4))
 (segment (start 117.05 34.1) (end 117 34.15) (width 0.2) (layer "F.Cu") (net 4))
 (segment (start 140 19.5) (end 140 30.5) (width 0.2) (layer "F.Cu") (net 4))
 (via (at 147.5 70) (size 0.6) (drill 0.3) (layers "F.Cu" "B.Cu") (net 4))
 (segment (start 143.5 65) (end 124.85 65) (width 0.2) (layer "B.Cu") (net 4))
 (segment (start 147.5 70) (end 147.5 69) (width 0.2) (layer "B.Cu") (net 4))
 (segment (start 147.5 69) (end 143.5 65) (width 0.2) (layer "B.Cu") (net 4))
 (segment (start 109.1 79) (end 134.92 79) (width 0.2) (layer "F.Cu") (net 3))
 (segment (start 119 29.5) (end 118.5 29.5) (width 0.2) (layer "F.Cu") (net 3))
 (segment (start 134.92 79) (end 136.38 77.54) (width 0.2) (layer "F.Cu") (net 3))
 (segment (start 116.35 31.65) (end 107 31.65) (width 0.2) (layer "F.Cu") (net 3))
 (segment (start 124.5 24) (end 119 29.5) (width 0.2) (layer "F.Cu") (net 3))
 (segment (start 126.4 22) (end 134.5 30.1) (width 0.2) (layer "F.Cu") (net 3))
 (segment (start 131.6 30.1) (end 134.5 30.1) (width 0.2) (layer "F.Cu") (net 3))
 (segment (start 130.5 30) (end 131.5 30) (width 0.2) (layer "F.Cu") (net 3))
 (segment (start 130.6 30.1) (end 130.5 30) (width 0.2) (layer "F.Cu") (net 3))
 (segment (start 131.5 30) (end 131.6 30.1) (width 0.2) (layer "F.Cu") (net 3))
 (segment (start 124.5 22) (end 126.4 22) (width 0.2) (layer "F.Cu") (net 3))
 (segment (start 124.5 22) (end 124.5 24) (width 0.2) (layer "F.Cu") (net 3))
 (segment (start 118.5 29.5) (end 116.35 31.65) (width 0.2) (layer "F.Cu") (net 3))
 (via (at 130.5 30) (size 0.6) (drill 0.3) (layers "F.Cu" "B.Cu") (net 3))
 (segment (start 135.5 63) (end 137 63) (width 0.2) (layer "B.Cu") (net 3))
 (segment (start 130.5 30) (end 130.5 58) (width 0.2) (layer "B.Cu") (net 3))
 (segment (start 130.5 58) (end 135.5 63) (width 0.2) (layer "B.Cu") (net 3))
 (segment (start 137 63) (end 125.294365 63) (width 0.2) (layer "B.Cu") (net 3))
 (segment (start 109.294365 79) (end 109.1 79) (width 0.2) (layer "B.Cu") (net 3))
 (segment (start 125.294365 63) (end 109.294365 79) (width 0.2) (layer "B.Cu") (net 3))
 (segment (start 162.43 40.08) (end 156.5 40.08) (width 0.2) (layer "F.Cu") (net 30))
 (segment (start 173.5 51.15) (end 162.43 40.08) (width 0.2) (layer "F.Cu") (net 30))
 (segment (start 161.65 63) (end 173.5 51.15) (width 0.2) (layer "F.Cu") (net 30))
 (segment (start 152 63) (end 161.65 63) (width 0.2) (layer "F.Cu") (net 30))
 (segment (start 141.85 88) (end 165.15 88) (width 0.2) (layer "F.Cu") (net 1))
 (segment (start 141.85 77.93) (end 136.38 72.46) (width 0.2) (layer "F.Cu") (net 1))
 (segment (start 141.85 88) (end 141.85 77.93) (width 0.2) (layer "F.Cu") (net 1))
 (segment (start 139.8 66.5) (end 136.38 69.92) (width 0.2) (layer "F.Cu") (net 2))
 (segment (start 177.85 68.2) (end 173.5 63.85) (width 0.2) (layer "F.Cu") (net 2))
 (segment (start 170.85 66.5) (end 139.8 66.5) (width 0.2) (layer "F.Cu") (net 2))
 (segment (start 177.85 88) (end 177.85 68.2) (width 0.2) (layer "F.Cu") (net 2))
 (segment (start 173.5 63.85) (end 170.85 66.5) (width 0.2) (layer "F.Cu") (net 2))
 (segment (start 112.15 65) (end 122.15 75) (width 0.2) (layer "F.Cu") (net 39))
 (segment (start 107 59.85) (end 112.15 65) (width 0.2) (layer "F.Cu") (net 39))
 (segment (start 107 44.35) (end 107 59.85) (width 0.2) (layer "F.Cu") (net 39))
 (segment (start 122.15 75) (end 136.38 75) (width 0.2) (layer "F.Cu") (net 39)))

